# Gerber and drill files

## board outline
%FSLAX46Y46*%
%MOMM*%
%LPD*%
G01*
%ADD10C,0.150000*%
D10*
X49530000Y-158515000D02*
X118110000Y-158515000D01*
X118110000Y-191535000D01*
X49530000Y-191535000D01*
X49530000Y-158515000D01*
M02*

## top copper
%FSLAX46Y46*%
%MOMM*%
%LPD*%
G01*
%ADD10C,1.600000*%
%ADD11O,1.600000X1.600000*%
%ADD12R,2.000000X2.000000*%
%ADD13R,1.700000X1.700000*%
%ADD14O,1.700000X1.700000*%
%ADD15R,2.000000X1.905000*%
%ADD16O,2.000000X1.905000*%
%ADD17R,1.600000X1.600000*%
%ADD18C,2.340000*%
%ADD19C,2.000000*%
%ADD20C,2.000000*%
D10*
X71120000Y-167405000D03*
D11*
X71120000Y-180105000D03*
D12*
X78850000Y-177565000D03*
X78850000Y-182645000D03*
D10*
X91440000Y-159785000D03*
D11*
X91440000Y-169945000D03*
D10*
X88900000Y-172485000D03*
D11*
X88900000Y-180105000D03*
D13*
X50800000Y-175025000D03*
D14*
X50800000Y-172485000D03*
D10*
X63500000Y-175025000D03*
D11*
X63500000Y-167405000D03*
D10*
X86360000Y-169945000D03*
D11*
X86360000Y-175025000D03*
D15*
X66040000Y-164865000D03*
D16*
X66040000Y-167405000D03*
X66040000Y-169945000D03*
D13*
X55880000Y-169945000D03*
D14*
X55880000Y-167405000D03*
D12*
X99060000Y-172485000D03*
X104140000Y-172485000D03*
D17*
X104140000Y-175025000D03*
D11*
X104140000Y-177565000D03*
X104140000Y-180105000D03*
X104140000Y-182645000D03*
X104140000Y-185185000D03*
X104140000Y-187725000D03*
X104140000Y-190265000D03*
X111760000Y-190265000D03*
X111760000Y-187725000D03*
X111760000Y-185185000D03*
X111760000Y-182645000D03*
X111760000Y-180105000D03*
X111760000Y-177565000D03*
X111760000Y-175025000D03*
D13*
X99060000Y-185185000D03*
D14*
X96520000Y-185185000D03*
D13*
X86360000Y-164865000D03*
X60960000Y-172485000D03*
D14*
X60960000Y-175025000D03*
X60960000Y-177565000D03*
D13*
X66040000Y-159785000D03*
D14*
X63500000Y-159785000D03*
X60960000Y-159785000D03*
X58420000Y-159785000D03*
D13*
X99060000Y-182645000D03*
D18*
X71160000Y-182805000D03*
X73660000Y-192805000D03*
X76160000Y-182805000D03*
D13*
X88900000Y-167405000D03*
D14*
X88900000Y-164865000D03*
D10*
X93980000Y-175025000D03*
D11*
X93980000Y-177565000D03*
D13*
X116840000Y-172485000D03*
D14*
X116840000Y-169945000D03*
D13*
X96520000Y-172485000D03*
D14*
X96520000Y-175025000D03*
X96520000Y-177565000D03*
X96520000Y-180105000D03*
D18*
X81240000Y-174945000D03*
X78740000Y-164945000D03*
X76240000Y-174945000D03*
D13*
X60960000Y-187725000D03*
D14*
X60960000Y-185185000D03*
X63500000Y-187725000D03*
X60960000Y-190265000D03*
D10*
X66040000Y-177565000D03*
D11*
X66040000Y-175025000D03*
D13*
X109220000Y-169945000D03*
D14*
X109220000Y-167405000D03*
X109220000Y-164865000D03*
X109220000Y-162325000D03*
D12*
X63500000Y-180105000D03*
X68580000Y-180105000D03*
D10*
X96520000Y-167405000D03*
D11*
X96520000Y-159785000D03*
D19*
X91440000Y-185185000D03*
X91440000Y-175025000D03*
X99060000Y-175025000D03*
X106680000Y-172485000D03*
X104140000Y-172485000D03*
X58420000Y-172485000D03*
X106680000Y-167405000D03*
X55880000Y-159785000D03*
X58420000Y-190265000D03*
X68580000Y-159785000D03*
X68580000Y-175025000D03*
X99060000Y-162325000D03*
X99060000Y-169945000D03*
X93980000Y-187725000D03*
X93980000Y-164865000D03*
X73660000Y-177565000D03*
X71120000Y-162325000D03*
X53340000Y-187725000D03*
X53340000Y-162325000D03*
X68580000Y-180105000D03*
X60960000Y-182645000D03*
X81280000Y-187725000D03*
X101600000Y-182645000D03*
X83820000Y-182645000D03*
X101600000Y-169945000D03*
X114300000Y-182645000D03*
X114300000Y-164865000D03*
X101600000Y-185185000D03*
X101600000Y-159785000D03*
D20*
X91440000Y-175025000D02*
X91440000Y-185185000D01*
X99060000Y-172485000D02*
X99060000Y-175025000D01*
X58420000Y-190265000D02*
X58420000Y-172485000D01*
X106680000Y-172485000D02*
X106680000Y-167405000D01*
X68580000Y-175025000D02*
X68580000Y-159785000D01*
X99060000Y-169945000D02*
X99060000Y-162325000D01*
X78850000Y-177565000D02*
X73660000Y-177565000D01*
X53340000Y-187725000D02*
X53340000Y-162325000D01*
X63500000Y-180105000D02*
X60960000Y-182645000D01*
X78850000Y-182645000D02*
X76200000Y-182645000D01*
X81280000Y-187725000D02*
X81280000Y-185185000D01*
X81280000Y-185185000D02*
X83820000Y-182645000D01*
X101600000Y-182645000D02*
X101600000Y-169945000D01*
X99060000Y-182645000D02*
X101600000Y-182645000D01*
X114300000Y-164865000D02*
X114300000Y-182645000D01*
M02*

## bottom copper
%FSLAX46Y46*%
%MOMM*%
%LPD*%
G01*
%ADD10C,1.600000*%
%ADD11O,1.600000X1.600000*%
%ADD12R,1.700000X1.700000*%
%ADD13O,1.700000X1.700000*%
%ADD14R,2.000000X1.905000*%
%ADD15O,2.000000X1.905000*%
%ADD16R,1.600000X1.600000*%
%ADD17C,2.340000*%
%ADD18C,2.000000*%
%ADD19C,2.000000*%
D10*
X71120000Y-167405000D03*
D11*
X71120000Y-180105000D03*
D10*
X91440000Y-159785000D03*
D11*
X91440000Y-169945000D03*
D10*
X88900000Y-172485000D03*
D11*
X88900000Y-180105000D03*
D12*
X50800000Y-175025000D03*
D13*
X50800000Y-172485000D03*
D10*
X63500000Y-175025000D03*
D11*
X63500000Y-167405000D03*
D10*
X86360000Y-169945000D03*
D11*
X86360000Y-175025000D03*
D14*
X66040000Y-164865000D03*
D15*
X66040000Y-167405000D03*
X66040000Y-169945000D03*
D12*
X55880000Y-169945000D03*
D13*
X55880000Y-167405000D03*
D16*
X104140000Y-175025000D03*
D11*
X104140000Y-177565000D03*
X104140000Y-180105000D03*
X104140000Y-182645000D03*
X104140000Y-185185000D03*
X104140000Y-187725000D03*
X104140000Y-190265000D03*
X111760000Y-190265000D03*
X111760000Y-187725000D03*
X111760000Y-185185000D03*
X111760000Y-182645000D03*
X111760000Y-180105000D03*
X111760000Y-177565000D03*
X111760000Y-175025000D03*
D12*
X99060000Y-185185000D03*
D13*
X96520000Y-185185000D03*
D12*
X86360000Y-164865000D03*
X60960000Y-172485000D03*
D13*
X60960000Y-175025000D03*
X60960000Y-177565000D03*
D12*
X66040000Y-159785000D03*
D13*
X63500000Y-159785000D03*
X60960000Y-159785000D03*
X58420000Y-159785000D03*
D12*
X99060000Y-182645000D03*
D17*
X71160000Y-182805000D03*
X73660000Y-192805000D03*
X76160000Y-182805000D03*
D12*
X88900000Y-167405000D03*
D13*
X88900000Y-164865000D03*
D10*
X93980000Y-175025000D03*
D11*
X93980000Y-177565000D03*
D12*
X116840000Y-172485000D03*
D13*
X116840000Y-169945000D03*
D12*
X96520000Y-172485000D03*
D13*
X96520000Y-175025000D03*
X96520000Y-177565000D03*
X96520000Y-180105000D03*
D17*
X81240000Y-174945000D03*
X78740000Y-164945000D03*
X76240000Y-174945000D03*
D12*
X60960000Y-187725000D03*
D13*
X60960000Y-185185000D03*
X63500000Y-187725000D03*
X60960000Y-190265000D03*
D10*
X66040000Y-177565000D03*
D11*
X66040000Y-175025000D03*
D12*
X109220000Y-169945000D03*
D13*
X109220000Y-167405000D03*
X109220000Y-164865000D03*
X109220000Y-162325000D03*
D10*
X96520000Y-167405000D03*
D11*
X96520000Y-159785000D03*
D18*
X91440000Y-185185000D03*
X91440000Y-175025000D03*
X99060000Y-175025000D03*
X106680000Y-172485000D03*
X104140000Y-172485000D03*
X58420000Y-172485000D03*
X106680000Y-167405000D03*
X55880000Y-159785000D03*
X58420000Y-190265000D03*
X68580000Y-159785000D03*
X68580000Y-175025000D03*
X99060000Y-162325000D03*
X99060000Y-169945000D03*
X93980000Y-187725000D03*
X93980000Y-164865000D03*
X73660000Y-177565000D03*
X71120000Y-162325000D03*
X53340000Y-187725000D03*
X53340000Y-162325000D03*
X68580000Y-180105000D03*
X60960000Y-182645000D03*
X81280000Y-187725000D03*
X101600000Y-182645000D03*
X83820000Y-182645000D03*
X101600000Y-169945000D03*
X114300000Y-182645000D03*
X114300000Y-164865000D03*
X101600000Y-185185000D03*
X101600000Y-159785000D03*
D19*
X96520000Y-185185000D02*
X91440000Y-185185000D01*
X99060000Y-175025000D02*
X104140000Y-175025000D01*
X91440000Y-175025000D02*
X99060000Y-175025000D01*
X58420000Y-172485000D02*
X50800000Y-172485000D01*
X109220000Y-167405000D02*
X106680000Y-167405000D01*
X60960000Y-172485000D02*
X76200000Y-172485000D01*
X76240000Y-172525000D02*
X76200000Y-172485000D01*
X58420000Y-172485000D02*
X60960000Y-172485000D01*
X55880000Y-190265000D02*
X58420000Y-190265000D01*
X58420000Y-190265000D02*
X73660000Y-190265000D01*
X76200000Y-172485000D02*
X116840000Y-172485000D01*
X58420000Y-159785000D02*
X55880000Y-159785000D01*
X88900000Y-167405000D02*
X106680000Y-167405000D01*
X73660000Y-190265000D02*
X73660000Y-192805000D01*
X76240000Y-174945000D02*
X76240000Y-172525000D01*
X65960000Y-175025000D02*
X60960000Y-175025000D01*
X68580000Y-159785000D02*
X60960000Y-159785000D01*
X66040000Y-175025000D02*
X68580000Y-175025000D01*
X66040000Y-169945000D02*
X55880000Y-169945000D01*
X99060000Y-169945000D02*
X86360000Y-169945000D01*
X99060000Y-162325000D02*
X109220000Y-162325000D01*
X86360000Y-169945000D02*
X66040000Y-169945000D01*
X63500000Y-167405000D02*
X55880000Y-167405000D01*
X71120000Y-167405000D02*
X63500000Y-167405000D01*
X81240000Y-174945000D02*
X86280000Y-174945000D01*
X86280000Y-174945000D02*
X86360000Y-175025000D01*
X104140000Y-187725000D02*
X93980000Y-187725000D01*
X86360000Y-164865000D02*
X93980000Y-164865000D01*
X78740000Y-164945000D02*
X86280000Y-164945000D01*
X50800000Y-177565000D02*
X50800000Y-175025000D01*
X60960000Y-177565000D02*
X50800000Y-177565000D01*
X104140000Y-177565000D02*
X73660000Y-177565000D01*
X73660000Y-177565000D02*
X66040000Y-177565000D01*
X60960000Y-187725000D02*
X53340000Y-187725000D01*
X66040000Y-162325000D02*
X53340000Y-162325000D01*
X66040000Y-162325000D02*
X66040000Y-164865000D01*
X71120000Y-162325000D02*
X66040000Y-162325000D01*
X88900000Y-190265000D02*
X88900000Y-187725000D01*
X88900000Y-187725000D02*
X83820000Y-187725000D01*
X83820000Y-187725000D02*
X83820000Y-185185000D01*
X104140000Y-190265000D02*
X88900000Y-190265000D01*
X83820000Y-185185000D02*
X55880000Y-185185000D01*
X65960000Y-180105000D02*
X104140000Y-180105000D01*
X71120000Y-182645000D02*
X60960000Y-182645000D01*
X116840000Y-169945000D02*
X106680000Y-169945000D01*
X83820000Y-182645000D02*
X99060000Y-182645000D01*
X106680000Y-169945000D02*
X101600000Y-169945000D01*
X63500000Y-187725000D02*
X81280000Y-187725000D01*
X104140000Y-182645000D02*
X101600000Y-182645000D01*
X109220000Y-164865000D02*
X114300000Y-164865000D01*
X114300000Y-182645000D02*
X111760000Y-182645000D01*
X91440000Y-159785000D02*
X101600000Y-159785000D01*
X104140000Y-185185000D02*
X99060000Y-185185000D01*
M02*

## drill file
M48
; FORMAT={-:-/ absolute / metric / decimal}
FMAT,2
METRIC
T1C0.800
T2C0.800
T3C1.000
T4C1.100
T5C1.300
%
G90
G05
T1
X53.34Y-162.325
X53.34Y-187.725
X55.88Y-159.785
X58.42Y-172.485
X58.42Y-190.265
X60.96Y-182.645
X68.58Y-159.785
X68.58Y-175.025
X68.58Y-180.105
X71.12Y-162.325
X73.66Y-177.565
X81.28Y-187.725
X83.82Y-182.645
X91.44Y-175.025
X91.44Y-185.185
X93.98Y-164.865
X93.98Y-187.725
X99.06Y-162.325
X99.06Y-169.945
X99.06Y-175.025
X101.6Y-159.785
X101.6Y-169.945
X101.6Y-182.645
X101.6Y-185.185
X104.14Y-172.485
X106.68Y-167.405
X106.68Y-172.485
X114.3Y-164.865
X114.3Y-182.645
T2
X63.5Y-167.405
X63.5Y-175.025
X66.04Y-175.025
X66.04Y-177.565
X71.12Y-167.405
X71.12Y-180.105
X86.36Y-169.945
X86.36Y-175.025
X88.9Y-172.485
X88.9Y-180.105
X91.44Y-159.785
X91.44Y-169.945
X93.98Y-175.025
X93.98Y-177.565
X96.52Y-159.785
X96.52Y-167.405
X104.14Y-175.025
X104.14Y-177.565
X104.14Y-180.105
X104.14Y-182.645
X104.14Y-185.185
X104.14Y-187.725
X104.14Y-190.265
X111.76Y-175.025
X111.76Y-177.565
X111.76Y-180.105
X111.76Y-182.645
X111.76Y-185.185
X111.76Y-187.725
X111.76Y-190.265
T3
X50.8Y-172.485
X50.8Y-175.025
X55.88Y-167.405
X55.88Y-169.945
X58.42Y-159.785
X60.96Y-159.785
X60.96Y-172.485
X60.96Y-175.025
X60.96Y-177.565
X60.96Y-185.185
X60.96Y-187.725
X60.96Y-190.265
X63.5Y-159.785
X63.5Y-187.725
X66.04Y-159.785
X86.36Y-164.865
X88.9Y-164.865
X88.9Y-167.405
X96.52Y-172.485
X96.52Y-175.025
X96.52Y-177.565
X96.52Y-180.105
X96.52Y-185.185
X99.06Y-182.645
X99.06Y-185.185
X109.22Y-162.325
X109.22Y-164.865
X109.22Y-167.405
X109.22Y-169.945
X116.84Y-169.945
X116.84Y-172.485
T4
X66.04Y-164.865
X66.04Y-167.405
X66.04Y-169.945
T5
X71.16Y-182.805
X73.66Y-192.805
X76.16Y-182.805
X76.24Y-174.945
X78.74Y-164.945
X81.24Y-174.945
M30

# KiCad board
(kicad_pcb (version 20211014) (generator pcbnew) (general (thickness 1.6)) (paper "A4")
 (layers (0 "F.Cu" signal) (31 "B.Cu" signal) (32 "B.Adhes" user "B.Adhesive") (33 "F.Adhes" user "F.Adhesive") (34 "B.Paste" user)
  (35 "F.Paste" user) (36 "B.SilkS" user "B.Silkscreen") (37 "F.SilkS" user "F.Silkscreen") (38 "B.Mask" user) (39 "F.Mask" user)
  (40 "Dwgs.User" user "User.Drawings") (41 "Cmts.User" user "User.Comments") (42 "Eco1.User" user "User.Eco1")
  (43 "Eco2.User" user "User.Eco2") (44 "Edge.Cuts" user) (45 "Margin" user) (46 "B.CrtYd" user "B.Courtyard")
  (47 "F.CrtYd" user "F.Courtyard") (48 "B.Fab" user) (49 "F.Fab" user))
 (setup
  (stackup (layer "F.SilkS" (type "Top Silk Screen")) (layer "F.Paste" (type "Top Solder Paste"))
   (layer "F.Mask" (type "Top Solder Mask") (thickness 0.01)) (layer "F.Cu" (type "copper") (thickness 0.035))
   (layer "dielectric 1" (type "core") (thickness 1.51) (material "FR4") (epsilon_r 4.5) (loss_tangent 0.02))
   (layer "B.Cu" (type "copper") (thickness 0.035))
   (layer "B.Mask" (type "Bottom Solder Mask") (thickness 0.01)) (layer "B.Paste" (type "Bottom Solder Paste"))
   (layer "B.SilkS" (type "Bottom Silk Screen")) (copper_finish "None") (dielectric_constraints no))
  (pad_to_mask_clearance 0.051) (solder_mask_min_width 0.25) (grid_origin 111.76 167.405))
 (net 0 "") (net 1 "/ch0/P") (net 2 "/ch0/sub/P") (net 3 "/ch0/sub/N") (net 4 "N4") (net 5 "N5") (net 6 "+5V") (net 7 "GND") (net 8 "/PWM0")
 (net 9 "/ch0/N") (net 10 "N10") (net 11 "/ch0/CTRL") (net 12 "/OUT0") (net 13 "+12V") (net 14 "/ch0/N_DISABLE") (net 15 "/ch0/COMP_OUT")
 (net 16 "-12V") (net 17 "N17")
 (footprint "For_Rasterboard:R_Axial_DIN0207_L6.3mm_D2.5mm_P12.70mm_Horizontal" (layer "F.Cu") (at 71.12 167.405 -90)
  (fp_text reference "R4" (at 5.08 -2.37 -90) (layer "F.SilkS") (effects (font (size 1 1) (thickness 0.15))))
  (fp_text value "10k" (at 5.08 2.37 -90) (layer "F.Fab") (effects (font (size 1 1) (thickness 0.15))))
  (pad "1" thru_hole circle (at 0 0 270) (size 1.6 1.6) (drill 0.8) (layers *.Cu *.Mask) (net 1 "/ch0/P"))
  (pad "2" thru_hole oval (at 12.7 0 270) (size 1.6 1.6) (drill 0.8) (layers *.Cu *.Mask) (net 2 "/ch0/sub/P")))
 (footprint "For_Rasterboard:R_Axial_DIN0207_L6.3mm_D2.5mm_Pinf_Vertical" (layer "F.Cu") (at 78.85 177.565 -90)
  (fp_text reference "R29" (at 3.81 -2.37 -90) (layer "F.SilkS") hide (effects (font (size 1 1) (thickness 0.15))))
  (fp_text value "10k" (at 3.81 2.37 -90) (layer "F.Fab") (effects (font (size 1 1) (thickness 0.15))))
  (pad "1" smd rect (at 0 0 270) (size 2 2) (layers "F.Cu") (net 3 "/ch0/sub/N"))
  (pad "2" smd rect (at 5.08 0 270) (size 2 2) (layers "F.Cu") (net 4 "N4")))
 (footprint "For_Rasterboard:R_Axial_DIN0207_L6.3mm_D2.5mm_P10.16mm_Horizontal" (layer "F.Cu") (at 91.44 159.785 -90)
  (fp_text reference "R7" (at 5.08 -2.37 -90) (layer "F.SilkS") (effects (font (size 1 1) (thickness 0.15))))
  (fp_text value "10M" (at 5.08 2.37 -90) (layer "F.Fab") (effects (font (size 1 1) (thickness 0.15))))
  (pad "1" thru_hole circle (at 0 0 270) (size 1.6 1.6) (drill 0.8) (layers *.Cu *.Mask) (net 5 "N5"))
  (pad "2" thru_hole oval (at 10.16 0 270) (size 1.6 1.6) (drill 0.8) (layers *.Cu *.Mask) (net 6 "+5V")))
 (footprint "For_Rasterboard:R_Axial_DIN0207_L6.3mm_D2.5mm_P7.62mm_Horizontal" (layer "F.Cu") (at 88.9 172.485 -90)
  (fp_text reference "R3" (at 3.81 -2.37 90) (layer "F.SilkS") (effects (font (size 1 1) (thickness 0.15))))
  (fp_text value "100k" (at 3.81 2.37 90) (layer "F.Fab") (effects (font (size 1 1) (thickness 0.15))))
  (pad "1" thru_hole circle (at 0 0 270) (size 1.6 1.6) (drill 0.8) (layers *.Cu *.Mask) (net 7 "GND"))
  (pad "2" thru_hole oval (at 7.62 0 270) (size 1.6 1.6) (drill 0.8) (layers *.Cu *.Mask) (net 2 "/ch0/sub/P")))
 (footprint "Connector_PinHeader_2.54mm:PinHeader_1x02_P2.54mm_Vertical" (layer "F.Cu") (at 50.8 175.025 180)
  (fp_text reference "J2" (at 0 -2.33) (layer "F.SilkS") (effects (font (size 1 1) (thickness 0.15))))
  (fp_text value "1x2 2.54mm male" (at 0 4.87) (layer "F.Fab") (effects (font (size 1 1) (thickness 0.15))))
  (pad "1" thru_hole rect (at 0 0 180) (size 1.7 1.7) (drill 1) (layers *.Cu *.Mask) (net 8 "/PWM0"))
  (pad "2" thru_hole oval (at 0 2.54 180) (size 1.7 1.7) (drill 1) (layers *.Cu *.Mask) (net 7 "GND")))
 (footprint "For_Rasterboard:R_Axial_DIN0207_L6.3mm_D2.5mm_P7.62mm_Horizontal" (layer "F.Cu") (at 63.5 175.025 90)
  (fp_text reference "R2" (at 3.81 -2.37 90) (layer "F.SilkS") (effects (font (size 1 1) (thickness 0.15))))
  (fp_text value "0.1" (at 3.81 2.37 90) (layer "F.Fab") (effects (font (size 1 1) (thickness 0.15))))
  (pad "1" thru_hole circle (at 0 0 90) (size 1.6 1.6) (drill 0.8) (layers *.Cu *.Mask) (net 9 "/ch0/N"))
  (pad "2" thru_hole oval (at 7.62 0 90) (size 1.6 1.6) (drill 0.8) (layers *.Cu *.Mask) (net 1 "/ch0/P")))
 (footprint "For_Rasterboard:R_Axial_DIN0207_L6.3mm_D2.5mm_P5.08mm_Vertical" (layer "F.Cu") (at 86.36 169.945 -90)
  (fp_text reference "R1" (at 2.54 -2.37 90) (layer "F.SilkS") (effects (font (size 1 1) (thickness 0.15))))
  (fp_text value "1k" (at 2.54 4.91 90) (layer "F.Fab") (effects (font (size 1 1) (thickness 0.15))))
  (pad "1" thru_hole circle (at 0 0 270) (size 1.6 1.6) (drill 0.8) (layers *.Cu *.Mask) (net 6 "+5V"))
  (pad "2" thru_hole oval (at 5.08 0 270) (size 1.6 1.6) (drill 0.8) (layers *.Cu *.Mask) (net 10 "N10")))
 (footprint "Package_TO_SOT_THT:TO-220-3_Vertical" (layer "F.Cu") (at 66.04 164.865 -90)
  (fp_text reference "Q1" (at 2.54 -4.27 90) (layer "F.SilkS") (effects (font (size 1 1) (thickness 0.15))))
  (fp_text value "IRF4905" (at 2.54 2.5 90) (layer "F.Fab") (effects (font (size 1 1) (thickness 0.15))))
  (pad "1" thru_hole rect (at 0 0 270) (size 1.905 2) (drill 1.1) (layers *.Cu *.Mask) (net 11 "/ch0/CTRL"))
  (pad "2" thru_hole oval (at 2.54 0 270) (size 1.905 2) (drill 1.1) (layers *.Cu *.Mask) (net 1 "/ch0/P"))
  (pad "3" thru_hole oval (at 5.08 0 270) (size 1.905 2) (drill 1.1) (layers *.Cu *.Mask) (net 6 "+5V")))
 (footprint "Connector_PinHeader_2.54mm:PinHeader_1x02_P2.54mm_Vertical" (layer "F.Cu") (at 55.88 169.945 180)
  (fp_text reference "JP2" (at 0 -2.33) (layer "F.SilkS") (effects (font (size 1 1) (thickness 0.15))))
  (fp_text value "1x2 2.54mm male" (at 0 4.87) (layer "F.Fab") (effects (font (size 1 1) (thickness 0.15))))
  (pad "1" thru_hole rect (at 0 0 180) (size 1.7 1.7) (drill 1) (layers *.Cu *.Mask) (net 6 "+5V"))
  (pad "2" thru_hole oval (at 0 2.54 180) (size 1.7 1.7) (drill 1) (layers *.Cu *.Mask) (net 1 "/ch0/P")))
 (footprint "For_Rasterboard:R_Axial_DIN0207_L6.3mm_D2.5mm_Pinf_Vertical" (layer "F.Cu") (at 99.06 172.485)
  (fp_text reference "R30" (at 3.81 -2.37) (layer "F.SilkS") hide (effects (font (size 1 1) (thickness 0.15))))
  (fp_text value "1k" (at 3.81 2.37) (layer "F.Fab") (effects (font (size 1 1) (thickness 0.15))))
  (pad "1" smd rect (at 0 0) (size 2 2) (layers "F.Cu") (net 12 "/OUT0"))
  (pad "2" smd rect (at 5.08 0) (size 2 2) (layers "F.Cu") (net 7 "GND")))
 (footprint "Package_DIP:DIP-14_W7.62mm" (layer "F.Cu") (at 104.14 175.025)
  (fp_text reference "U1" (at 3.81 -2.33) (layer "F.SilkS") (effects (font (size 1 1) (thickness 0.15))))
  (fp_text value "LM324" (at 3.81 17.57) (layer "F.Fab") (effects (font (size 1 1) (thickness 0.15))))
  (pad "1" thru_hole rect (at 0 0) (size 1.6 1.6) (drill 0.8) (layers *.Cu *.Mask) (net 12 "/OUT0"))
  (pad "2" thru_hole oval (at 0 2.54) (size 1.6 1.6) (drill 0.8) (layers *.Cu *.Mask) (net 3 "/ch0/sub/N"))
  (pad "3" thru_hole oval (at 0 5.08) (size 1.6 1.6) (drill 0.8) (layers *.Cu *.Mask) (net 2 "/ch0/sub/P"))
  (pad "4" thru_hole oval (at 0 7.62) (size 1.6 1.6) (drill 0.8) (layers *.Cu *.Mask) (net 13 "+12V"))
  (pad "5" thru_hole oval (at 0 10.16) (size 1.6 1.6) (drill 0.8) (layers *.Cu *.Mask) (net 5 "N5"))
  (pad "6" thru_hole oval (at 0 12.7) (size 1.6 1.6) (drill 0.8) (layers *.Cu *.Mask) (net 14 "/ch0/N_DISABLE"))
  (pad "7" thru_hole oval (at 0 15.24) (size 1.6 1.6) (drill 0.8) (layers *.Cu *.Mask) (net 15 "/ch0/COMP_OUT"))
  (pad "8" thru_hole oval (at 7.62 15.24) (size 1.6 1.6) (drill 0.8) (layers *.Cu *.Mask))
  (pad "9" thru_hole oval (at 7.62 12.7) (size 1.6 1.6) (drill 0.8) (layers *.Cu *.Mask))
  (pad "10" thru_hole oval (at 7.62 10.16) (size 1.6 1.6) (drill 0.8) (layers *.Cu *.Mask))
  (pad "11" thru_hole oval (at 7.62 7.62) (size 1.6 1.6) (drill 0.8) (layers *.Cu *.Mask) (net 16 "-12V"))
  (pad "12" thru_hole oval (at 7.62 5.08) (size 1.6 1.6) (drill 0.8) (layers *.Cu *.Mask))
  (pad "13" thru_hole oval (at 7.62 2.54) (size 1.6 1.6) (drill 0.8) (layers *.Cu *.Mask))
  (pad "14" thru_hole oval (at 7.62 0) (size 1.6 1.6) (drill 0.8) (layers *.Cu *.Mask)))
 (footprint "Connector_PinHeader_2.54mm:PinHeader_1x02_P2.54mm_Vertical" (layer "F.Cu") (at 99.06 185.185 -90)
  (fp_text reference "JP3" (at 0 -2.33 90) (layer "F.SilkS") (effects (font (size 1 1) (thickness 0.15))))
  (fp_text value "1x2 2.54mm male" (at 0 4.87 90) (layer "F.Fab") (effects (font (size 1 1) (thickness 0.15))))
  (pad "1" thru_hole rect (at 0 0 270) (size 1.7 1.7) (drill 1) (layers *.Cu *.Mask) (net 5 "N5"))
  (pad "2" thru_hole oval (at 0 2.54 270) (size 1.7 1.7) (drill 1) (layers *.Cu *.Mask) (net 12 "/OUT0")))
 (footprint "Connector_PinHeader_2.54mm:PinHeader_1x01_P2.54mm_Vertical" (layer "F.Cu") (at 86.36 164.865)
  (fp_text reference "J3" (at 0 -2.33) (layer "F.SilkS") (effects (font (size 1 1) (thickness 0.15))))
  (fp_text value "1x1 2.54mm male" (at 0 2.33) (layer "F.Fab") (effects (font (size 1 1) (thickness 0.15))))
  (pad "1" thru_hole rect (at 0 0) (size 1.7 1.7) (drill 1) (layers *.Cu *.Mask) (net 14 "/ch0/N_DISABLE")))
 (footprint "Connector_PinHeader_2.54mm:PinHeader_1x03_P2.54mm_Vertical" (layer "F.Cu") (at 60.96 172.485)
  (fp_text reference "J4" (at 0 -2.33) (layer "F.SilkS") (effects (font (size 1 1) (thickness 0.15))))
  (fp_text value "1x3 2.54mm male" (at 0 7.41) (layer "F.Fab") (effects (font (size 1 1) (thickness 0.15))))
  (pad "1" thru_hole rect (at 0 0) (size 1.7 1.7) (drill 1) (layers *.Cu *.Mask) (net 7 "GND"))
  (pad "2" thru_hole oval (at 0 2.54) (size 1.7 1.7) (drill 1) (layers *.Cu *.Mask) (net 9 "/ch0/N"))
  (pad "3" thru_hole oval (at 0 5.08) (size 1.7 1.7) (drill 1) (layers *.Cu *.Mask) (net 8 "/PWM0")))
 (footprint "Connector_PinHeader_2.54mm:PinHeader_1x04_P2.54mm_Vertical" (layer "F.Cu") (at 66.04 159.785 -90)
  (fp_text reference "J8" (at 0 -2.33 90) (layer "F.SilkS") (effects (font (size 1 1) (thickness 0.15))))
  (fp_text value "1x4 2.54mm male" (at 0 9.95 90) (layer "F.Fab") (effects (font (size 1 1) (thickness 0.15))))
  (pad "1" thru_hole rect (at 0 0 270) (size 1.7 1.7) (drill 1) (layers *.Cu *.Mask) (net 9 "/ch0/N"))
  (pad "2" thru_hole oval (at 0 2.54 270) (size 1.7 1.7) (drill 1) (layers *.Cu *.Mask) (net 9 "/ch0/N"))
  (pad "3" thru_hole oval (at 0 5.08 270) (size 1.7 1.7) (drill 1) (layers *.Cu *.Mask) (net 9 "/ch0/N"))
  (pad "4" thru_hole oval (at 0 7.62 270) (size 1.7 1.7) (drill 1) (layers *.Cu *.Mask) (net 7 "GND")))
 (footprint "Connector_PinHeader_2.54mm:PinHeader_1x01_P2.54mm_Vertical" (layer "F.Cu") (at 99.06 182.645)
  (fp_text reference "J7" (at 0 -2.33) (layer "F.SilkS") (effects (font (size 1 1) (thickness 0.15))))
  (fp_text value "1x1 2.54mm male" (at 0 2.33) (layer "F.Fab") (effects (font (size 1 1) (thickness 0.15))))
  (pad "1" thru_hole rect (at 0 0) (size 1.7 1.7) (drill 1) (layers *.Cu *.Mask) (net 13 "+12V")))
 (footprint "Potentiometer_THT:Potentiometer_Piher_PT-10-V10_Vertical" (layer "F.Cu") (at 71.16 182.805 -90)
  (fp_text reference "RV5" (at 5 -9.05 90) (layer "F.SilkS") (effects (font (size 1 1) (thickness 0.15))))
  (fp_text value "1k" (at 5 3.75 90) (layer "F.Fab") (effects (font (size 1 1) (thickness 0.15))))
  (pad "1" thru_hole circle (at 0 0 270) (size 2.34 2.34) (drill 1.3) (layers *.Cu *.Mask) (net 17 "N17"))
  (pad "2" thru_hole circle (at 10 -2.5 270) (size 2.34 2.34) (drill 1.3) (layers *.Cu *.Mask) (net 7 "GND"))
  (pad "3" thru_hole circle (at 0 -5 270) (size 2.34 2.34) (drill 1.3) (layers *.Cu *.Mask) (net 4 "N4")))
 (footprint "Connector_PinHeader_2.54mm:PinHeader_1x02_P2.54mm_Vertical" (layer "F.Cu") (at 88.9 167.405 180)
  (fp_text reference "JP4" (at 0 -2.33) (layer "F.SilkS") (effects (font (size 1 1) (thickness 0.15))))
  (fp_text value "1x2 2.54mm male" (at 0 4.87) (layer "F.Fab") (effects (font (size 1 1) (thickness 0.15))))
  (pad "1" thru_hole rect (at 0 0 180) (size 1.7 1.7) (drill 1) (layers *.Cu *.Mask) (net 7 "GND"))
  (pad "2" thru_hole oval (at 0 2.54 180) (size 1.7 1.7) (drill 1) (layers *.Cu *.Mask) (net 14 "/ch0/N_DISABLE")))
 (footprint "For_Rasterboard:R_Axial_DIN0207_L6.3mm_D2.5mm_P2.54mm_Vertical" (layer "F.Cu") (at 93.98 175.025 -90)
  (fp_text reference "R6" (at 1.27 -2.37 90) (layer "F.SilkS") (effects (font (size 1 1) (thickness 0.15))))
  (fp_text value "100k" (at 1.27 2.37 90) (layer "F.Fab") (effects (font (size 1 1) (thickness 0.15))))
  (pad "1" thru_hole circle (at 0 0 270) (size 1.6 1.6) (drill 0.8) (layers *.Cu *.Mask) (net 12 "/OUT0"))
  (pad "2" thru_hole oval (at 2.54 0 270) (size 1.6 1.6) (drill 0.8) (layers *.Cu *.Mask) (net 3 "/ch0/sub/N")))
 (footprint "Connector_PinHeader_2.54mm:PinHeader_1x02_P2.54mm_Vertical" (layer "F.Cu") (at 116.84 172.485 180)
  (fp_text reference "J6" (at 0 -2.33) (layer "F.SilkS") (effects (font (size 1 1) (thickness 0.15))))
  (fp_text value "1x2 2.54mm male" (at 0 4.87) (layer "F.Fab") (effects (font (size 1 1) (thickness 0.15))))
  (pad "1" thru_hole rect (at 0 0 180) (size 1.7 1.7) (drill 1) (layers *.Cu *.Mask) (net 7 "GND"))
  (pad "2" thru_hole oval (at 0 2.54 180) (size 1.7 1.7) (drill 1) (layers *.Cu *.Mask) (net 13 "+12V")))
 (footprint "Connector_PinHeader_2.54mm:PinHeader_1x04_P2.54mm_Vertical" (layer "F.Cu") (at 96.52 172.485)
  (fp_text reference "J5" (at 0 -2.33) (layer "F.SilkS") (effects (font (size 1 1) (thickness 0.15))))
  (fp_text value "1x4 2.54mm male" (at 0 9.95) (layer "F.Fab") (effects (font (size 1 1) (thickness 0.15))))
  (pad "1" thru_hole rect (at 0 0) (size 1.7 1.7) (drill 1) (layers *.Cu *.Mask) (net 7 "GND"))
  (pad "2" thru_hole oval (at 0 2.54) (size 1.7 1.7) (drill 1) (layers *.Cu *.Mask) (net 12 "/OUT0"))
  (pad "3" thru_hole oval (at 0 5.08) (size 1.7 1.7) (drill 1) (layers *.Cu *.Mask) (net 3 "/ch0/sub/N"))
  (pad "4" thru_hole oval (at 0 7.62) (size 1.7 1.7) (drill 1) (layers *.Cu *.Mask) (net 2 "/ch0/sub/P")))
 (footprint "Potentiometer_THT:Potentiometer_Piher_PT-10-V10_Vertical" (layer "F.Cu") (at 81.24 174.945 90)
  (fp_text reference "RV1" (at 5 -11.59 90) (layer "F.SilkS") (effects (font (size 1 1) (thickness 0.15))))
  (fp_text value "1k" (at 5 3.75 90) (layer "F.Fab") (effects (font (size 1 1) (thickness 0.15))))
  (pad "1" thru_hole circle (at 0 0 90) (size 2.34 2.34) (drill 1.3) (layers *.Cu *.Mask) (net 10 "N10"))
  (pad "2" thru_hole circle (at 10 -2.5 90) (size 2.34 2.34) (drill 1.3) (layers *.Cu *.Mask) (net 14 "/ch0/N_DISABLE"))
  (pad "3" thru_hole circle (at 0 -5 90) (size 2.34 2.34) (drill 1.3) (layers *.Cu *.Mask) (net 7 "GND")))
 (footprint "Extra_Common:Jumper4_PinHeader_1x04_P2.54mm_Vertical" (layer "F.Cu") (at 60.96 187.725)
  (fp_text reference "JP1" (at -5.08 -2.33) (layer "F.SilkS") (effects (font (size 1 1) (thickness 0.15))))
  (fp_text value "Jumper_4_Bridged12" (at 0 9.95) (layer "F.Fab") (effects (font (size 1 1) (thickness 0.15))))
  (pad "1" thru_hole rect (at 0 0) (size 1.7 1.7) (drill 1) (layers *.Cu *.Mask) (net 11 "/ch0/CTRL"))
  (pad "2" thru_hole oval (at 0 -2.54) (size 1.7 1.7) (drill 1) (layers *.Cu *.Mask) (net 15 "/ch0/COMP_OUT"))
  (pad "3" thru_hole oval (at 2.54 0) (size 1.7 1.7) (drill 1) (layers *.Cu *.Mask) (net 13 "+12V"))
  (pad "4" thru_hole oval (at 0 2.54) (size 1.7 1.7) (drill 1) (layers *.Cu *.Mask) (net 7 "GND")))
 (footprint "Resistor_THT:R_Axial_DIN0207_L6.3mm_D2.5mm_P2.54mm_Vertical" (layer "F.Cu") (at 66.04 177.565 90)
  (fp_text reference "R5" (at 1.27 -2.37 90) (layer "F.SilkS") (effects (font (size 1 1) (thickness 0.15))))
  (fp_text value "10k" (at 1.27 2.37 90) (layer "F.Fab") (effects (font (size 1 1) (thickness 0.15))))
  (pad "1" thru_hole circle (at 0 0 90) (size 1.6 1.6) (drill 0.8) (layers *.Cu *.Mask) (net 3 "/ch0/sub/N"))
  (pad "2" thru_hole oval (at 2.54 0 90) (size 1.6 1.6) (drill 0.8) (layers *.Cu *.Mask) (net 9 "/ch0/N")))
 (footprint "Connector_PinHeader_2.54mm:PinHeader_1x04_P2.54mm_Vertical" (layer "F.Cu") (at 109.22 169.945 180)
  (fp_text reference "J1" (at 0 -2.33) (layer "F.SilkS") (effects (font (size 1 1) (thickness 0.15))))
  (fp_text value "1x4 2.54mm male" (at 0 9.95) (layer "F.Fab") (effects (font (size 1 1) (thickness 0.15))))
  (pad "1" thru_hole rect (at 0 0 180) (size 1.7 1.7) (drill 1) (layers *.Cu *.Mask) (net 13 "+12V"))
  (pad "2" thru_hole oval (at 0 2.54 180) (size 1.7 1.7) (drill 1) (layers *.Cu *.Mask) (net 7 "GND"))
  (pad "3" thru_hole oval (at 0 5.08 180) (size 1.7 1.7) (drill 1) (layers *.Cu *.Mask) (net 16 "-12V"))
  (pad "4" thru_hole oval (at 0 7.62 180) (size 1.7 1.7) (drill 1) (layers *.Cu *.Mask) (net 6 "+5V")))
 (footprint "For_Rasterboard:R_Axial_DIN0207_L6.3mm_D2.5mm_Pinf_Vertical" (layer "F.Cu") (at 63.5 180.105)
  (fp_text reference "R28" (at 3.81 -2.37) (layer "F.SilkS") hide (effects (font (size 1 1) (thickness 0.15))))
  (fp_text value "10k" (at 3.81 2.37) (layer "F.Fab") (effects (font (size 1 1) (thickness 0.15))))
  (pad "1" smd rect (at 0 0) (size 2 2) (layers "F.Cu") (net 17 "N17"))
  (pad "2" smd rect (at 5.08 0) (size 2 2) (layers "F.Cu") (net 2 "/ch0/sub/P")))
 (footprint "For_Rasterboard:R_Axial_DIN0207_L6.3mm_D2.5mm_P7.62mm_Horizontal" (layer "F.Cu") (at 96.52 167.405 90)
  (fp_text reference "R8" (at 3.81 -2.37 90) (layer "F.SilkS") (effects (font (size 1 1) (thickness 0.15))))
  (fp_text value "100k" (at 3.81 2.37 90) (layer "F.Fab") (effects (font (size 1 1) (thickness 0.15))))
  (pad "1" thru_hole circle (at 0 0 90) (size 1.6 1.6) (drill 0.8) (layers *.Cu *.Mask) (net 7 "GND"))
  (pad "2" thru_hole oval (at 7.62 0 90) (size 1.6 1.6) (drill 0.8) (layers *.Cu *.Mask) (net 5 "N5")))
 (gr_rect (start 118.11 191.535) (end 49.53 158.515) (layer "Edge.Cuts") (width 0.15) (fill none))
 (segment (start 91.44 175.025) (end 91.44 185.185) (width 2) (layer "F.Cu") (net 12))
 (segment (start 99.06 172.485) (end 99.06 175.025) (width 2) (layer "F.Cu") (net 12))
 (via (at 91.44 185.185) (size 2) (drill 0.8) (layers "F.Cu" "B.Cu") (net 12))
 (via (at 91.44 175.025) (size 2) (drill 0.8) (layers "F.Cu" "B.Cu") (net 12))
 (via (at 99.06 175.025) (size 2) (drill 0.8) (layers "F.Cu" "B.Cu") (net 12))
 (segment (start 96.52 185.185) (end 91.44 185.185) (width 2) (layer "B.Cu") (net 12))
 (segment (start 99.06 175.025) (end 104.14 175.025) (width 2) (layer "B.Cu") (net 12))
 (segment (start 91.44 175.025) (end 99.06 175.025) (width 2) (layer "B.Cu") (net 12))
 (segment (start 58.42 190.265) (end 58.42 172.485) (width 2) (layer "F.Cu") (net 7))
 (segment (start 106.68 172.485) (end 106.68 167.405) (width 2) (layer "F.Cu") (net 7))
 (via (at 106.68 172.485) (size 2) (drill 0.8) (layers "F.Cu" "B.Cu") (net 7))
 (via (at 104.14 172.485) (size 2) (drill 0.8) (layers "F.Cu" "B.Cu") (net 7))
 (via (at 58.42 172.485) (size 2) (drill 0.8) (layers "F.Cu" "B.Cu") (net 7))
 (via (at 106.68 167.405) (size 2) (drill 0.8) (layers "F.Cu" "B.Cu") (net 7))
 (via (at 55.88 159.785) (size 2) (drill 0.8) (layers "F.Cu" "B.Cu") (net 7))
 (via (at 58.42 190.265) (size 2) (drill 0.8) (layers "F.Cu" "B.Cu") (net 7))
 (segment (start 58.42 172.485) (end 50.8 172.485) (width 2) (layer "B.Cu") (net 7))
 (segment (start 109.22 167.405) (end 106.68 167.405) (width 2) (layer "B.Cu") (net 7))
 (segment (start 60.96 172.485) (end 76.2 172.485) (width 2) (layer "B.Cu") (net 7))
 (segment (start 76.24 172.525) (end 76.2 172.485) (width 2) (layer "B.Cu") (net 7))
 (segment (start 58.42 172.485) (end 60.96 172.485) (width 2) (layer "B.Cu") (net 7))
 (segment (start 55.88 190.265) (end 58.42 190.265) (width 2) (layer "B.Cu") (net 7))
 (segment (start 58.42 190.265) (end 73.66 190.265) (width 2) (layer "B.Cu") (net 7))
 (segment (start 76.2 172.485) (end 116.84 172.485) (width 2) (layer "B.Cu") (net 7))
 (segment (start 58.42 159.785) (end 55.88 159.785) (width 2) (layer "B.Cu") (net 7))
 (segment (start 88.9 167.405) (end 106.68 167.405) (width 2) (layer "B.Cu") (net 7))
 (segment (start 73.66 190.265) (end 73.66 192.805) (width 2) (layer "B.Cu") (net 7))
 (segment (start 76.24 174.945) (end 76.24 172.525) (width 2) (layer "B.Cu") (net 7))
 (segment (start 68.58 175.025) (end 68.58 159.785) (width 2) (layer "F.Cu") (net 9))
 (via (at 68.58 159.785) (size 2) (drill 0.8) (layers "F.Cu" "B.Cu") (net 9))
 (via (at 68.58 175.025) (size 2) (drill 0.8) (layers "F.Cu" "B.Cu") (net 9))
 (segment (start 65.96 175.025) (end 60.96 175.025) (width 2) (layer "B.Cu") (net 9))
 (segment (start 68.58 159.785) (end 60.96 159.785) (width 2) (layer "B.Cu") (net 9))
 (segment (start 66.04 175.025) (end 68.58 175.025) (width 2) (layer "B.Cu") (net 9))
 (segment (start 99.06 169.945) (end 99.06 162.325) (width 2) (layer "F.Cu") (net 6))
 (via (at 99.06 162.325) (size 2) (drill 0.8) (layers "F.Cu" "B.Cu") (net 6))
 (via (at 99.06 169.945) (size 2) (drill 0.8) (layers "F.Cu" "B.Cu") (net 6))
 (segment (start 66.04 169.945) (end 55.88 169.945) (width 2) (layer "B.Cu") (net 6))
 (segment (start 99.06 169.945) (end 86.36 169.945) (width 2) (layer "B.Cu") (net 6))
 (segment (start 99.06 162.325) (end 109.22 162.325) (width 2) (layer "B.Cu") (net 6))
 (segment (start 86.36 169.945) (end 66.04 169.945) (width 2) (layer "B.Cu") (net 6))
 (segment (start 63.5 167.405) (end 55.88 167.405) (width 2) (layer "B.Cu") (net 1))
 (segment (start 71.12 167.405) (end 63.5 167.405) (width 2) (layer "B.Cu") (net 1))
 (segment (start 81.24 174.945) (end 86.28 174.945) (width 2) (layer "B.Cu") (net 10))
 (segment (start 86.28 174.945) (end 86.36 175.025) (width 2) (layer "B.Cu") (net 10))
 (via (at 93.98 187.725) (size 2) (drill 0.8) (layers "F.Cu" "B.Cu") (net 14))
 (via (at 93.98 164.865) (size 2) (drill 0.8) (layers "F.Cu" "B.Cu") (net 14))
 (segment (start 104.14 187.725) (end 93.98 187.725) (width 2) (layer "B.Cu") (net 14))
 (segment (start 86.36 164.865) (end 93.98 164.865) (width 2) (layer "B.Cu") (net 14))
 (segment (start 78.74 164.945) (end 86.28 164.945) (width 2) (layer "B.Cu") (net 14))
 (segment (start 50.8 177.565) (end 50.8 175.025) (width 2) (layer "B.Cu") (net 8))
 (segment (start 60.96 177.565) (end 50.8 177.565) (width 2) (layer "B.Cu") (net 8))
 (segment (start 78.85 177.565) (end 73.66 177.565) (width 2) (layer "F.Cu") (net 3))
 (via (at 73.66 177.565) (size 2) (drill 0.8) (layers "F.Cu" "B.Cu") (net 3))
 (segment (start 104.14 177.565) (end 73.66 177.565) (width 2) (layer "B.Cu") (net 3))
 (segment (start 73.66 177.565) (end 66.04 177.565) (width 2) (layer "B.Cu") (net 3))
 (segment (start 53.34 187.725) (end 53.34 162.325) (width 2) (layer "F.Cu") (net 11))
 (via (at 71.12 162.325) (size 2) (drill 0.8) (layers "F.Cu" "B.Cu") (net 11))
 (via (at 53.34 187.725) (size 2) (drill 0.8) (layers "F.Cu" "B.Cu") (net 11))
 (via (at 53.34 162.325) (size 2) (drill 0.8) (layers "F.Cu" "B.Cu") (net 11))
 (segment (start 60.96 187.725) (end 53.34 187.725) (width 2) (layer "B.Cu") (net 11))
 (segment (start 66.04 162.325) (end 53.34 162.325) (width 2) (layer "B.Cu") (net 11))
 (segment (start 66.04 162.325) (end 66.04 164.865) (width 2) (layer "B.Cu") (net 11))
 (segment (start 71.12 162.325) (end 66.04 162.325) (width 2) (layer "B.Cu") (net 11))
 (segment (start 88.9 190.265) (end 88.9 187.725) (width 2) (layer "B.Cu") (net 15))
 (segment (start 88.9 187.725) (end 83.82 187.725) (width 2) (layer "B.Cu") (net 15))
 (segment (start 83.82 187.725) (end 83.82 185.185) (width 2) (layer "B.Cu") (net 15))
 (segment (start 104.14 190.265) (end 88.9 190.265) (width 2) (layer "B.Cu") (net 15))
 (segment (start 83.82 185.185) (end 55.88 185.185) (width 2) (layer "B.Cu") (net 15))
 (via (at 68.58 180.105) (size 2) (drill 0.8) (layers "F.Cu" "B.Cu") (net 2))
 (segment (start 65.96 180.105) (end 104.14 180.105) (width 2) (layer "B.Cu") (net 2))
 (segment (start 63.5 180.105) (end 60.96 182.645) (width 2) (layer "F.Cu") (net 17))
 (via (at 60.96 182.645) (size 2) (drill 0.8) (layers "F.Cu" "B.Cu") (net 17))
 (segment (start 71.12 182.645) (end 60.96 182.645) (width 2) (layer "B.Cu") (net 17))
 (segment (start 78.85 182.645) (end 76.2 182.645) (width 2) (layer "F.Cu") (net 4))
 (segment (start 81.28 187.725) (end 81.28 185.185) (width 2) (layer "F.Cu") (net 13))
 (segment (start 81.28 185.185) (end 83.82 182.645) (width 2) (layer "F.Cu") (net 13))
 (segment (start 101.6 182.645) (end 101.6 169.945) (width 2) (layer "F.Cu") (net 13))
 (segment (start 99.06 182.645) (end 101.6 182.645) (width 2) (layer "F.Cu") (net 13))
 (via (at 81.28 187.725) (size 2) (drill 0.8) (layers "F.Cu" "B.Cu") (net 13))
 (via (at 101.6 182.645) (size 2) (drill 0.8) (layers "F.Cu" "B.Cu") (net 13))
 (via (at 83.82 182.645) (size 2) (drill 0.8) (layers "F.Cu" "B.Cu") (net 13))
 (via (at 101.6 169.945) (size 2) (drill 0.8) (layers "F.Cu" "B.Cu") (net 13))
 (segment (start 116.84 169.945) (end 106.68 169.945) (width 2) (layer "B.Cu") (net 13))
 (segment (start 83.82 182.645) (end 99.06 182.645) (width 2) (layer "B.Cu") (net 13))
 (segment (start 106.68 169.945) (end 101.6 169.945) (width 2) (layer "B.Cu") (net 13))
 (segment (start 63.5 187.725) (end 81.28 187.725) (width 2) (layer "B.Cu") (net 13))
 (segment (start 104.14 182.645) (end 101.6 182.645) (width 2) (layer "B.Cu") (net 13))
 (segment (start 114.3 164.865) (end 114.3 182.645) (width 2) (layer "F.Cu") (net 16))
 (via (at 114.3 182.645) (size 2) (drill 0.8) (layers "F.Cu" "B.Cu") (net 16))
 (via (at 114.3 164.865) (size 2) (drill 0.8) (layers "F.Cu" "B.Cu") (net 16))
 (segment (start 109.22 164.865) (end 114.3 164.865) (width 2) (layer "B.Cu") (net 16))
 (segment (start 114.3 182.645) (end 111.76 182.645) (width 2) (layer "B.Cu") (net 16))
 (via (at 101.6 185.185) (size 2) (drill 0.8) (layers "F.Cu" "B.Cu") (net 5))
 (via (at 101.6 159.785) (size 2) (drill 0.8) (layers "F.Cu" "B.Cu") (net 5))
 (segment (start 91.44 159.785) (end 101.6 159.785) (width 2) (layer "B.Cu") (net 5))
 (segment (start 104.14 185.185) (end 99.06 185.185) (width 2) (layer "B.Cu") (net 5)))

